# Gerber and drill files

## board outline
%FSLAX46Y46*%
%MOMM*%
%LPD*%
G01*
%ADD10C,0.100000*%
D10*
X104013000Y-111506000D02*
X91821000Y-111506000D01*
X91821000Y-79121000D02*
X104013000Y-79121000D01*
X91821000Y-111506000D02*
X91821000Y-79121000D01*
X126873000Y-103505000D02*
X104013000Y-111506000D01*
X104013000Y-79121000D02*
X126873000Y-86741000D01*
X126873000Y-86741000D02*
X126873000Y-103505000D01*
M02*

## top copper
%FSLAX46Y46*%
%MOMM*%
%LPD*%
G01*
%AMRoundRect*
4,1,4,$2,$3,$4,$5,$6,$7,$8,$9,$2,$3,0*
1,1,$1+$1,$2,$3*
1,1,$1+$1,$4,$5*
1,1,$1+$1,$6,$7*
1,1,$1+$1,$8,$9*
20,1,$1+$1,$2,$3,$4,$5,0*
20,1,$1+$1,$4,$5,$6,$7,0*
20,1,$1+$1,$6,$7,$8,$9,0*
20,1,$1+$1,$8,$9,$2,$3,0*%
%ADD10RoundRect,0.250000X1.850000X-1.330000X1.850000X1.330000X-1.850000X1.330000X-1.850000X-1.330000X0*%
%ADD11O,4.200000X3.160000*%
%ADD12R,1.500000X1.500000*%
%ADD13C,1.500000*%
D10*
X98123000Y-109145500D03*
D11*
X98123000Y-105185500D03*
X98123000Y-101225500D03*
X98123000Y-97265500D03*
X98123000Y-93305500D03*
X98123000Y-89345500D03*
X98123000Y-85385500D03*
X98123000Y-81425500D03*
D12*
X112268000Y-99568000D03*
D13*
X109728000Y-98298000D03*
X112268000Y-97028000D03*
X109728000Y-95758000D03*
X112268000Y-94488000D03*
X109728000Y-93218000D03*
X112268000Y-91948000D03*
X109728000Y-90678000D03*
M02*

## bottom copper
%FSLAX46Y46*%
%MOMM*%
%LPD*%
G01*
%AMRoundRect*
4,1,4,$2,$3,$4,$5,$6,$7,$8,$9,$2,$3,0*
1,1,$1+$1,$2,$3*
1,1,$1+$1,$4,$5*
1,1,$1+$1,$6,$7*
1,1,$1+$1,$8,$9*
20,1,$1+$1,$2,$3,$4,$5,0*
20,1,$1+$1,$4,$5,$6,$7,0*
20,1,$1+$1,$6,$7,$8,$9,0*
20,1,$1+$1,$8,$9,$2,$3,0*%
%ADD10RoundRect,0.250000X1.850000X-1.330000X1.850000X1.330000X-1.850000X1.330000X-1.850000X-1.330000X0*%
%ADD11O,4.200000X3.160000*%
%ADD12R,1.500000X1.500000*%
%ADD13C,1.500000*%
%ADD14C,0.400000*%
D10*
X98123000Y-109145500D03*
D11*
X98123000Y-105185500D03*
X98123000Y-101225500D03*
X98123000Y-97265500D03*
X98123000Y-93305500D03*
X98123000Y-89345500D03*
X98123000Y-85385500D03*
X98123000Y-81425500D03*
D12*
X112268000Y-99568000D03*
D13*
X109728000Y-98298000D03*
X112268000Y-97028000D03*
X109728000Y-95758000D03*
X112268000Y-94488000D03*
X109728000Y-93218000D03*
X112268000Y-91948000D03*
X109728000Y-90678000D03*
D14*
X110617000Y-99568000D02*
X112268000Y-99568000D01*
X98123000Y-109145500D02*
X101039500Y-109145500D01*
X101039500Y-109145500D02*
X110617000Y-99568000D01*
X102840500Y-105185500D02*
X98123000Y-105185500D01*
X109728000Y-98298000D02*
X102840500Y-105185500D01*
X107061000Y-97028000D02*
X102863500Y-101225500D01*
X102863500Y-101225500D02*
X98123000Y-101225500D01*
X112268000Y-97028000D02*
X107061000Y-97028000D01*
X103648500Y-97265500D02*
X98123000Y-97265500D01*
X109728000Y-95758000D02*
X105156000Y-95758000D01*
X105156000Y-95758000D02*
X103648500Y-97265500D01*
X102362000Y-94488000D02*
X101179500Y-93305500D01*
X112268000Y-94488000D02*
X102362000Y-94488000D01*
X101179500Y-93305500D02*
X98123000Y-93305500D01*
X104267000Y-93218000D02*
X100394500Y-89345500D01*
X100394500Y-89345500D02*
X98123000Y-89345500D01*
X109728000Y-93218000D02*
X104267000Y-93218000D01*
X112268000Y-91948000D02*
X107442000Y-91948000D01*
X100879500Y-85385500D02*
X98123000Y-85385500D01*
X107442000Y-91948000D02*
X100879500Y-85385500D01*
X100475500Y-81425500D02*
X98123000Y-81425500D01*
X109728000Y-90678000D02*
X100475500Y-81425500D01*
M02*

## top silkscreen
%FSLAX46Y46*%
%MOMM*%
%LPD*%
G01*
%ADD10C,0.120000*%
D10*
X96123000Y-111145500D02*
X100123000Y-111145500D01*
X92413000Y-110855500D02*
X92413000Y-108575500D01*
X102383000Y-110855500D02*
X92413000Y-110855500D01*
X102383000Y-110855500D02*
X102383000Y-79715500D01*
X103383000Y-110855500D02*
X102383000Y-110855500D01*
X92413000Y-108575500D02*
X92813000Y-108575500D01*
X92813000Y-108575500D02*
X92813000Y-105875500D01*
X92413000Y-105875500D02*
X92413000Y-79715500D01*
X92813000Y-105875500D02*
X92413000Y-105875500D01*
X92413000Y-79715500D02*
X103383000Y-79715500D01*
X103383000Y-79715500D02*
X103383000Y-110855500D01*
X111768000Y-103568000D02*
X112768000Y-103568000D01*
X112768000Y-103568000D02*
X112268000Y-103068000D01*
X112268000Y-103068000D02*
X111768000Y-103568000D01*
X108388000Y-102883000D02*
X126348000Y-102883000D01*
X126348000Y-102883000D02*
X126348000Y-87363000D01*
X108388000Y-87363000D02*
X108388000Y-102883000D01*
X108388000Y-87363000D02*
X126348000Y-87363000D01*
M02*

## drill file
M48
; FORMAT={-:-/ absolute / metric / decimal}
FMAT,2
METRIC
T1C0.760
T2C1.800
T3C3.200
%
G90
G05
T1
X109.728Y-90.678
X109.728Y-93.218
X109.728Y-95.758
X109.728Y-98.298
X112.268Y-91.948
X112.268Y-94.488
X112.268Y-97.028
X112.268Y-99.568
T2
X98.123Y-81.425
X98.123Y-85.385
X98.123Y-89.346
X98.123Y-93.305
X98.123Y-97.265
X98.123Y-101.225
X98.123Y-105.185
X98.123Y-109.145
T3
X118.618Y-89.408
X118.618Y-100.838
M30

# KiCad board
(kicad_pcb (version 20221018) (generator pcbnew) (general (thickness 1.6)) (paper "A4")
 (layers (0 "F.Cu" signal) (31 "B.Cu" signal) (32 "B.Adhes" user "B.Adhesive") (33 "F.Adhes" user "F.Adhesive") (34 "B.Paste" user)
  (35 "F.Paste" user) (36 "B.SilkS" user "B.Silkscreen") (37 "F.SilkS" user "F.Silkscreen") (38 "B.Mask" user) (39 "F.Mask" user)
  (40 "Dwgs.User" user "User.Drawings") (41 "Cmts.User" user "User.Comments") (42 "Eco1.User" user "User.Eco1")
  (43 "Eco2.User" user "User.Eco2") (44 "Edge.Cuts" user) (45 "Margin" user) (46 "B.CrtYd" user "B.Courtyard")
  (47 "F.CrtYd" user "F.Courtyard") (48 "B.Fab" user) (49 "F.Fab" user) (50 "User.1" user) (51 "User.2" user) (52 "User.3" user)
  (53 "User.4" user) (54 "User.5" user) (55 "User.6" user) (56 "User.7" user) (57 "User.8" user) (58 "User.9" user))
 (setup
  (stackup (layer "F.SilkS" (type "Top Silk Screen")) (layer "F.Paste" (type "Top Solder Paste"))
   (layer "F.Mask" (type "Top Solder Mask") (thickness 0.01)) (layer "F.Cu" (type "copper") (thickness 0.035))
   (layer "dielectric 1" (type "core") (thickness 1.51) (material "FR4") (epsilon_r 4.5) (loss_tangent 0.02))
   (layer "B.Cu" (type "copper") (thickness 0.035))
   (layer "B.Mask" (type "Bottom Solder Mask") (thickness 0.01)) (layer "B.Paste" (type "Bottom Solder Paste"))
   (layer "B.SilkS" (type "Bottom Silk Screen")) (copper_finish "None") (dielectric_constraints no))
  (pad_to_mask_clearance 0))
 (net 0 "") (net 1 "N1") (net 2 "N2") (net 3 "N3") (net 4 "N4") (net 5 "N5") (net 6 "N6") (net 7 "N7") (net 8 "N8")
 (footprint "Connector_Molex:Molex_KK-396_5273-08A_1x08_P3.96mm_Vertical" (layer "F.Cu") (at 98.123 109.1455 90)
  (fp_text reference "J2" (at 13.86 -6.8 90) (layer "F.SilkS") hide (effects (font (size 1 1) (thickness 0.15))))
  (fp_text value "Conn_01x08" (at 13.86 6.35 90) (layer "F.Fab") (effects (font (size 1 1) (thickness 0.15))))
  (fp_line (start -2 -2) (end -2 2) (stroke (width 0.12) (type solid)) (layer "F.SilkS"))
  (fp_line (start -1.71 -5.71) (end 0.57 -5.71) (stroke (width 0.12) (type solid)) (layer "F.SilkS"))
  (fp_line (start -1.71 4.26) (end -1.71 -5.71) (stroke (width 0.12) (type solid)) (layer "F.SilkS"))
  (fp_line (start -1.71 4.26) (end 29.43 4.26) (stroke (width 0.12) (type solid)) (layer "F.SilkS"))
  (fp_line (start -1.71 5.26) (end -1.71 4.26) (stroke (width 0.12) (type solid)) (layer "F.SilkS"))
  (fp_line (start 0.57 -5.71) (end 0.57 -5.31) (stroke (width 0.12) (type solid)) (layer "F.SilkS"))
  (fp_line (start 0.57 -5.31) (end 3.27 -5.31) (stroke (width 0.12) (type solid)) (layer "F.SilkS"))
  (fp_line (start 3.27 -5.71) (end 29.43 -5.71) (stroke (width 0.12) (type solid)) (layer "F.SilkS"))
  (fp_line (start 3.27 -5.31) (end 3.27 -5.71) (stroke (width 0.12) (type solid)) (layer "F.SilkS"))
  (fp_line (start 29.43 -5.71) (end 29.43 5.26) (stroke (width 0.12) (type solid)) (layer "F.SilkS"))
  (fp_line (start 29.43 5.26) (end -1.71 5.26) (stroke (width 0.12) (type solid)) (layer "F.SilkS"))
  (pad "1" thru_hole roundrect (at 0 0 90) (size 3.16 4.2) (drill 1.8) (layers "*.Cu" "*.Mask") (roundrect_rratio 0.079114) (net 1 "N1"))
  (pad "2" thru_hole oval (at 3.96 0 90) (size 3.16 4.2) (drill 1.8) (layers "*.Cu" "*.Mask") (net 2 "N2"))
  (pad "3" thru_hole oval (at 7.92 0 90) (size 3.16 4.2) (drill 1.8) (layers "*.Cu" "*.Mask") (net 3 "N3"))
  (pad "4" thru_hole oval (at 11.88 0 90) (size 3.16 4.2) (drill 1.8) (layers "*.Cu" "*.Mask") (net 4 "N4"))
  (pad "5" thru_hole oval (at 15.84 0 90) (size 3.16 4.2) (drill 1.8) (layers "*.Cu" "*.Mask") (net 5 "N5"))
  (pad "6" thru_hole oval (at 19.8 0 90) (size 3.16 4.2) (drill 1.8) (layers "*.Cu" "*.Mask") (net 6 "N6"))
  (pad "7" thru_hole oval (at 23.76 0 90) (size 3.16 4.2) (drill 1.8) (layers "*.Cu" "*.Mask") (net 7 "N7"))
  (pad "8" thru_hole oval (at 27.72 0 90) (size 3.16 4.2) (drill 1.8) (layers "*.Cu" "*.Mask") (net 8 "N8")))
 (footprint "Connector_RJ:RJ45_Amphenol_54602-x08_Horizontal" (layer "F.Cu") (at 112.268 99.568 90)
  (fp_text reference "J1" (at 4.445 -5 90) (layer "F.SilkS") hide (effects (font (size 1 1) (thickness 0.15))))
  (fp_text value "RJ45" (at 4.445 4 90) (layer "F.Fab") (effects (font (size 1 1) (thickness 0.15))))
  (fp_line (start -4 -0.5) (end -4 0.5) (stroke (width 0.12) (type solid)) (layer "F.SilkS"))
  (fp_line (start -4 0.5) (end -3.5 0) (stroke (width 0.12) (type solid)) (layer "F.SilkS"))
  (fp_line (start -3.5 0) (end -4 -0.5) (stroke (width 0.12) (type solid)) (layer "F.SilkS"))
  (fp_line (start -3.315 -3.88) (end -3.315 14.08) (stroke (width 0.12) (type solid)) (layer "F.SilkS"))
  (fp_line (start -3.315 14.08) (end 12.205 14.08) (stroke (width 0.12) (type solid)) (layer "F.SilkS"))
  (fp_line (start 12.205 -3.88) (end -3.315 -3.88) (stroke (width 0.12) (type solid)) (layer "F.SilkS"))
  (fp_line (start 12.205 -3.88) (end 12.205 14.08) (stroke (width 0.12) (type solid)) (layer "F.SilkS"))
  (pad "" np_thru_hole circle (at -1.27 6.35 90) (size 3.2 3.2) (drill 3.2) (layers "*.Cu" "*.Mask"))
  (pad "" np_thru_hole circle (at 10.16 6.35 90) (size 3.2 3.2) (drill 3.2) (layers "*.Cu" "*.Mask"))
  (pad "1" thru_hole rect (at 0 0 90) (size 1.5 1.5) (drill 0.76) (layers "*.Cu" "*.Mask") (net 1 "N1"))
  (pad "2" thru_hole circle (at 1.27 -2.54 90) (size 1.5 1.5) (drill 0.76) (layers "*.Cu" "*.Mask") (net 2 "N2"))
  (pad "3" thru_hole circle (at 2.54 0 90) (size 1.5 1.5) (drill 0.76) (layers "*.Cu" "*.Mask") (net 3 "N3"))
  (pad "4" thru_hole circle (at 3.81 -2.54 90) (size 1.5 1.5) (drill 0.76) (layers "*.Cu" "*.Mask") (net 4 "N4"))
  (pad "5" thru_hole circle (at 5.08 0 90) (size 1.5 1.5) (drill 0.76) (layers "*.Cu" "*.Mask") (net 5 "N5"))
  (pad "6" thru_hole circle (at 6.35 -2.54 90) (size 1.5 1.5) (drill 0.76) (layers "*.Cu" "*.Mask") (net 6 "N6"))
  (pad "7" thru_hole circle (at 7.62 0 90) (size 1.5 1.5) (drill 0.76) (layers "*.Cu" "*.Mask") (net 7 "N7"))
  (pad "8" thru_hole circle (at 8.89 -2.54 90) (size 1.5 1.5) (drill 0.76) (layers "*.Cu" "*.Mask") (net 8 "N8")))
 (gr_line (start 104.013 111.506) (end 91.821 111.506) (stroke (width 0.1) (type default)) (layer "Edge.Cuts"))
 (gr_line (start 91.821 79.121) (end 104.013 79.121) (stroke (width 0.1) (type default)) (layer "Edge.Cuts"))
 (gr_line (start 91.821 111.506) (end 91.821 79.121) (stroke (width 0.1) (type default)) (layer "Edge.Cuts"))
 (gr_line (start 126.873 103.505) (end 104.013 111.506) (stroke (width 0.1) (type default)) (layer "Edge.Cuts"))
 (gr_line (start 104.013 79.121) (end 126.873 86.741) (stroke (width 0.1) (type default)) (layer "Edge.Cuts"))
 (gr_line (start 126.873 86.741) (end 126.873 103.505) (stroke (width 0.1) (type default)) (layer "Edge.Cuts"))
 (segment (start 110.617 99.568) (end 112.268 99.568) (width 0.4) (layer "B.Cu") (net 1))
 (segment (start 98.123 109.1455) (end 101.0395 109.1455) (width 0.4) (layer "B.Cu") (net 1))
 (segment (start 101.0395 109.1455) (end 110.617 99.568) (width 0.4) (layer "B.Cu") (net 1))
 (segment (start 102.8405 105.1855) (end 98.123 105.1855) (width 0.4) (layer "B.Cu") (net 2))
 (segment (start 109.728 98.298) (end 102.8405 105.1855) (width 0.4) (layer "B.Cu") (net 2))
 (segment (start 107.061 97.028) (end 102.8635 101.2255) (width 0.4) (layer "B.Cu") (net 3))
 (segment (start 102.8635 101.2255) (end 98.123 101.2255) (width 0.4) (layer "B.Cu") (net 3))
 (segment (start 112.268 97.028) (end 107.061 97.028) (width 0.4) (layer "B.Cu") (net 3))
 (segment (start 103.6485 97.2655) (end 98.123 97.2655) (width 0.4) (layer "B.Cu") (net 4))
 (segment (start 109.728 95.758) (end 105.156 95.758) (width 0.4) (layer "B.Cu") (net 4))
 (segment (start 105.156 95.758) (end 103.6485 97.2655) (width 0.4) (layer "B.Cu") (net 4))
 (segment (start 102.362 94.488) (end 101.1795 93.3055) (width 0.4) (layer "B.Cu") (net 5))
 (segment (start 112.268 94.488) (end 102.362 94.488) (width 0.4) (layer "B.Cu") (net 5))
 (segment (start 101.1795 93.3055) (end 98.123 93.3055) (width 0.4) (layer "B.Cu") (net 5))
 (segment (start 104.267 93.218) (end 100.3945 89.3455) (width 0.4) (layer "B.Cu") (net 6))
 (segment (start 100.3945 89.3455) (end 98.123 89.3455) (width 0.4) (layer "B.Cu") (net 6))
 (segment (start 109.728 93.218) (end 104.267 93.218) (width 0.4) (layer "B.Cu") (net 6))
 (segment (start 112.268 91.948) (end 107.442 91.948) (width 0.4) (layer "B.Cu") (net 7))
 (segment (start 100.8795 85.3855) (end 98.123 85.3855) (width 0.4) (layer "B.Cu") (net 7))
 (segment (start 107.442 91.948) (end 100.8795 85.3855) (width 0.4) (layer "B.Cu") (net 7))
 (segment (start 100.4755 81.4255) (end 98.123 81.4255) (width 0.4) (layer "B.Cu") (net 8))
 (segment (start 109.728 90.678) (end 100.4755 81.4255) (width 0.4) (layer "B.Cu") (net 8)))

